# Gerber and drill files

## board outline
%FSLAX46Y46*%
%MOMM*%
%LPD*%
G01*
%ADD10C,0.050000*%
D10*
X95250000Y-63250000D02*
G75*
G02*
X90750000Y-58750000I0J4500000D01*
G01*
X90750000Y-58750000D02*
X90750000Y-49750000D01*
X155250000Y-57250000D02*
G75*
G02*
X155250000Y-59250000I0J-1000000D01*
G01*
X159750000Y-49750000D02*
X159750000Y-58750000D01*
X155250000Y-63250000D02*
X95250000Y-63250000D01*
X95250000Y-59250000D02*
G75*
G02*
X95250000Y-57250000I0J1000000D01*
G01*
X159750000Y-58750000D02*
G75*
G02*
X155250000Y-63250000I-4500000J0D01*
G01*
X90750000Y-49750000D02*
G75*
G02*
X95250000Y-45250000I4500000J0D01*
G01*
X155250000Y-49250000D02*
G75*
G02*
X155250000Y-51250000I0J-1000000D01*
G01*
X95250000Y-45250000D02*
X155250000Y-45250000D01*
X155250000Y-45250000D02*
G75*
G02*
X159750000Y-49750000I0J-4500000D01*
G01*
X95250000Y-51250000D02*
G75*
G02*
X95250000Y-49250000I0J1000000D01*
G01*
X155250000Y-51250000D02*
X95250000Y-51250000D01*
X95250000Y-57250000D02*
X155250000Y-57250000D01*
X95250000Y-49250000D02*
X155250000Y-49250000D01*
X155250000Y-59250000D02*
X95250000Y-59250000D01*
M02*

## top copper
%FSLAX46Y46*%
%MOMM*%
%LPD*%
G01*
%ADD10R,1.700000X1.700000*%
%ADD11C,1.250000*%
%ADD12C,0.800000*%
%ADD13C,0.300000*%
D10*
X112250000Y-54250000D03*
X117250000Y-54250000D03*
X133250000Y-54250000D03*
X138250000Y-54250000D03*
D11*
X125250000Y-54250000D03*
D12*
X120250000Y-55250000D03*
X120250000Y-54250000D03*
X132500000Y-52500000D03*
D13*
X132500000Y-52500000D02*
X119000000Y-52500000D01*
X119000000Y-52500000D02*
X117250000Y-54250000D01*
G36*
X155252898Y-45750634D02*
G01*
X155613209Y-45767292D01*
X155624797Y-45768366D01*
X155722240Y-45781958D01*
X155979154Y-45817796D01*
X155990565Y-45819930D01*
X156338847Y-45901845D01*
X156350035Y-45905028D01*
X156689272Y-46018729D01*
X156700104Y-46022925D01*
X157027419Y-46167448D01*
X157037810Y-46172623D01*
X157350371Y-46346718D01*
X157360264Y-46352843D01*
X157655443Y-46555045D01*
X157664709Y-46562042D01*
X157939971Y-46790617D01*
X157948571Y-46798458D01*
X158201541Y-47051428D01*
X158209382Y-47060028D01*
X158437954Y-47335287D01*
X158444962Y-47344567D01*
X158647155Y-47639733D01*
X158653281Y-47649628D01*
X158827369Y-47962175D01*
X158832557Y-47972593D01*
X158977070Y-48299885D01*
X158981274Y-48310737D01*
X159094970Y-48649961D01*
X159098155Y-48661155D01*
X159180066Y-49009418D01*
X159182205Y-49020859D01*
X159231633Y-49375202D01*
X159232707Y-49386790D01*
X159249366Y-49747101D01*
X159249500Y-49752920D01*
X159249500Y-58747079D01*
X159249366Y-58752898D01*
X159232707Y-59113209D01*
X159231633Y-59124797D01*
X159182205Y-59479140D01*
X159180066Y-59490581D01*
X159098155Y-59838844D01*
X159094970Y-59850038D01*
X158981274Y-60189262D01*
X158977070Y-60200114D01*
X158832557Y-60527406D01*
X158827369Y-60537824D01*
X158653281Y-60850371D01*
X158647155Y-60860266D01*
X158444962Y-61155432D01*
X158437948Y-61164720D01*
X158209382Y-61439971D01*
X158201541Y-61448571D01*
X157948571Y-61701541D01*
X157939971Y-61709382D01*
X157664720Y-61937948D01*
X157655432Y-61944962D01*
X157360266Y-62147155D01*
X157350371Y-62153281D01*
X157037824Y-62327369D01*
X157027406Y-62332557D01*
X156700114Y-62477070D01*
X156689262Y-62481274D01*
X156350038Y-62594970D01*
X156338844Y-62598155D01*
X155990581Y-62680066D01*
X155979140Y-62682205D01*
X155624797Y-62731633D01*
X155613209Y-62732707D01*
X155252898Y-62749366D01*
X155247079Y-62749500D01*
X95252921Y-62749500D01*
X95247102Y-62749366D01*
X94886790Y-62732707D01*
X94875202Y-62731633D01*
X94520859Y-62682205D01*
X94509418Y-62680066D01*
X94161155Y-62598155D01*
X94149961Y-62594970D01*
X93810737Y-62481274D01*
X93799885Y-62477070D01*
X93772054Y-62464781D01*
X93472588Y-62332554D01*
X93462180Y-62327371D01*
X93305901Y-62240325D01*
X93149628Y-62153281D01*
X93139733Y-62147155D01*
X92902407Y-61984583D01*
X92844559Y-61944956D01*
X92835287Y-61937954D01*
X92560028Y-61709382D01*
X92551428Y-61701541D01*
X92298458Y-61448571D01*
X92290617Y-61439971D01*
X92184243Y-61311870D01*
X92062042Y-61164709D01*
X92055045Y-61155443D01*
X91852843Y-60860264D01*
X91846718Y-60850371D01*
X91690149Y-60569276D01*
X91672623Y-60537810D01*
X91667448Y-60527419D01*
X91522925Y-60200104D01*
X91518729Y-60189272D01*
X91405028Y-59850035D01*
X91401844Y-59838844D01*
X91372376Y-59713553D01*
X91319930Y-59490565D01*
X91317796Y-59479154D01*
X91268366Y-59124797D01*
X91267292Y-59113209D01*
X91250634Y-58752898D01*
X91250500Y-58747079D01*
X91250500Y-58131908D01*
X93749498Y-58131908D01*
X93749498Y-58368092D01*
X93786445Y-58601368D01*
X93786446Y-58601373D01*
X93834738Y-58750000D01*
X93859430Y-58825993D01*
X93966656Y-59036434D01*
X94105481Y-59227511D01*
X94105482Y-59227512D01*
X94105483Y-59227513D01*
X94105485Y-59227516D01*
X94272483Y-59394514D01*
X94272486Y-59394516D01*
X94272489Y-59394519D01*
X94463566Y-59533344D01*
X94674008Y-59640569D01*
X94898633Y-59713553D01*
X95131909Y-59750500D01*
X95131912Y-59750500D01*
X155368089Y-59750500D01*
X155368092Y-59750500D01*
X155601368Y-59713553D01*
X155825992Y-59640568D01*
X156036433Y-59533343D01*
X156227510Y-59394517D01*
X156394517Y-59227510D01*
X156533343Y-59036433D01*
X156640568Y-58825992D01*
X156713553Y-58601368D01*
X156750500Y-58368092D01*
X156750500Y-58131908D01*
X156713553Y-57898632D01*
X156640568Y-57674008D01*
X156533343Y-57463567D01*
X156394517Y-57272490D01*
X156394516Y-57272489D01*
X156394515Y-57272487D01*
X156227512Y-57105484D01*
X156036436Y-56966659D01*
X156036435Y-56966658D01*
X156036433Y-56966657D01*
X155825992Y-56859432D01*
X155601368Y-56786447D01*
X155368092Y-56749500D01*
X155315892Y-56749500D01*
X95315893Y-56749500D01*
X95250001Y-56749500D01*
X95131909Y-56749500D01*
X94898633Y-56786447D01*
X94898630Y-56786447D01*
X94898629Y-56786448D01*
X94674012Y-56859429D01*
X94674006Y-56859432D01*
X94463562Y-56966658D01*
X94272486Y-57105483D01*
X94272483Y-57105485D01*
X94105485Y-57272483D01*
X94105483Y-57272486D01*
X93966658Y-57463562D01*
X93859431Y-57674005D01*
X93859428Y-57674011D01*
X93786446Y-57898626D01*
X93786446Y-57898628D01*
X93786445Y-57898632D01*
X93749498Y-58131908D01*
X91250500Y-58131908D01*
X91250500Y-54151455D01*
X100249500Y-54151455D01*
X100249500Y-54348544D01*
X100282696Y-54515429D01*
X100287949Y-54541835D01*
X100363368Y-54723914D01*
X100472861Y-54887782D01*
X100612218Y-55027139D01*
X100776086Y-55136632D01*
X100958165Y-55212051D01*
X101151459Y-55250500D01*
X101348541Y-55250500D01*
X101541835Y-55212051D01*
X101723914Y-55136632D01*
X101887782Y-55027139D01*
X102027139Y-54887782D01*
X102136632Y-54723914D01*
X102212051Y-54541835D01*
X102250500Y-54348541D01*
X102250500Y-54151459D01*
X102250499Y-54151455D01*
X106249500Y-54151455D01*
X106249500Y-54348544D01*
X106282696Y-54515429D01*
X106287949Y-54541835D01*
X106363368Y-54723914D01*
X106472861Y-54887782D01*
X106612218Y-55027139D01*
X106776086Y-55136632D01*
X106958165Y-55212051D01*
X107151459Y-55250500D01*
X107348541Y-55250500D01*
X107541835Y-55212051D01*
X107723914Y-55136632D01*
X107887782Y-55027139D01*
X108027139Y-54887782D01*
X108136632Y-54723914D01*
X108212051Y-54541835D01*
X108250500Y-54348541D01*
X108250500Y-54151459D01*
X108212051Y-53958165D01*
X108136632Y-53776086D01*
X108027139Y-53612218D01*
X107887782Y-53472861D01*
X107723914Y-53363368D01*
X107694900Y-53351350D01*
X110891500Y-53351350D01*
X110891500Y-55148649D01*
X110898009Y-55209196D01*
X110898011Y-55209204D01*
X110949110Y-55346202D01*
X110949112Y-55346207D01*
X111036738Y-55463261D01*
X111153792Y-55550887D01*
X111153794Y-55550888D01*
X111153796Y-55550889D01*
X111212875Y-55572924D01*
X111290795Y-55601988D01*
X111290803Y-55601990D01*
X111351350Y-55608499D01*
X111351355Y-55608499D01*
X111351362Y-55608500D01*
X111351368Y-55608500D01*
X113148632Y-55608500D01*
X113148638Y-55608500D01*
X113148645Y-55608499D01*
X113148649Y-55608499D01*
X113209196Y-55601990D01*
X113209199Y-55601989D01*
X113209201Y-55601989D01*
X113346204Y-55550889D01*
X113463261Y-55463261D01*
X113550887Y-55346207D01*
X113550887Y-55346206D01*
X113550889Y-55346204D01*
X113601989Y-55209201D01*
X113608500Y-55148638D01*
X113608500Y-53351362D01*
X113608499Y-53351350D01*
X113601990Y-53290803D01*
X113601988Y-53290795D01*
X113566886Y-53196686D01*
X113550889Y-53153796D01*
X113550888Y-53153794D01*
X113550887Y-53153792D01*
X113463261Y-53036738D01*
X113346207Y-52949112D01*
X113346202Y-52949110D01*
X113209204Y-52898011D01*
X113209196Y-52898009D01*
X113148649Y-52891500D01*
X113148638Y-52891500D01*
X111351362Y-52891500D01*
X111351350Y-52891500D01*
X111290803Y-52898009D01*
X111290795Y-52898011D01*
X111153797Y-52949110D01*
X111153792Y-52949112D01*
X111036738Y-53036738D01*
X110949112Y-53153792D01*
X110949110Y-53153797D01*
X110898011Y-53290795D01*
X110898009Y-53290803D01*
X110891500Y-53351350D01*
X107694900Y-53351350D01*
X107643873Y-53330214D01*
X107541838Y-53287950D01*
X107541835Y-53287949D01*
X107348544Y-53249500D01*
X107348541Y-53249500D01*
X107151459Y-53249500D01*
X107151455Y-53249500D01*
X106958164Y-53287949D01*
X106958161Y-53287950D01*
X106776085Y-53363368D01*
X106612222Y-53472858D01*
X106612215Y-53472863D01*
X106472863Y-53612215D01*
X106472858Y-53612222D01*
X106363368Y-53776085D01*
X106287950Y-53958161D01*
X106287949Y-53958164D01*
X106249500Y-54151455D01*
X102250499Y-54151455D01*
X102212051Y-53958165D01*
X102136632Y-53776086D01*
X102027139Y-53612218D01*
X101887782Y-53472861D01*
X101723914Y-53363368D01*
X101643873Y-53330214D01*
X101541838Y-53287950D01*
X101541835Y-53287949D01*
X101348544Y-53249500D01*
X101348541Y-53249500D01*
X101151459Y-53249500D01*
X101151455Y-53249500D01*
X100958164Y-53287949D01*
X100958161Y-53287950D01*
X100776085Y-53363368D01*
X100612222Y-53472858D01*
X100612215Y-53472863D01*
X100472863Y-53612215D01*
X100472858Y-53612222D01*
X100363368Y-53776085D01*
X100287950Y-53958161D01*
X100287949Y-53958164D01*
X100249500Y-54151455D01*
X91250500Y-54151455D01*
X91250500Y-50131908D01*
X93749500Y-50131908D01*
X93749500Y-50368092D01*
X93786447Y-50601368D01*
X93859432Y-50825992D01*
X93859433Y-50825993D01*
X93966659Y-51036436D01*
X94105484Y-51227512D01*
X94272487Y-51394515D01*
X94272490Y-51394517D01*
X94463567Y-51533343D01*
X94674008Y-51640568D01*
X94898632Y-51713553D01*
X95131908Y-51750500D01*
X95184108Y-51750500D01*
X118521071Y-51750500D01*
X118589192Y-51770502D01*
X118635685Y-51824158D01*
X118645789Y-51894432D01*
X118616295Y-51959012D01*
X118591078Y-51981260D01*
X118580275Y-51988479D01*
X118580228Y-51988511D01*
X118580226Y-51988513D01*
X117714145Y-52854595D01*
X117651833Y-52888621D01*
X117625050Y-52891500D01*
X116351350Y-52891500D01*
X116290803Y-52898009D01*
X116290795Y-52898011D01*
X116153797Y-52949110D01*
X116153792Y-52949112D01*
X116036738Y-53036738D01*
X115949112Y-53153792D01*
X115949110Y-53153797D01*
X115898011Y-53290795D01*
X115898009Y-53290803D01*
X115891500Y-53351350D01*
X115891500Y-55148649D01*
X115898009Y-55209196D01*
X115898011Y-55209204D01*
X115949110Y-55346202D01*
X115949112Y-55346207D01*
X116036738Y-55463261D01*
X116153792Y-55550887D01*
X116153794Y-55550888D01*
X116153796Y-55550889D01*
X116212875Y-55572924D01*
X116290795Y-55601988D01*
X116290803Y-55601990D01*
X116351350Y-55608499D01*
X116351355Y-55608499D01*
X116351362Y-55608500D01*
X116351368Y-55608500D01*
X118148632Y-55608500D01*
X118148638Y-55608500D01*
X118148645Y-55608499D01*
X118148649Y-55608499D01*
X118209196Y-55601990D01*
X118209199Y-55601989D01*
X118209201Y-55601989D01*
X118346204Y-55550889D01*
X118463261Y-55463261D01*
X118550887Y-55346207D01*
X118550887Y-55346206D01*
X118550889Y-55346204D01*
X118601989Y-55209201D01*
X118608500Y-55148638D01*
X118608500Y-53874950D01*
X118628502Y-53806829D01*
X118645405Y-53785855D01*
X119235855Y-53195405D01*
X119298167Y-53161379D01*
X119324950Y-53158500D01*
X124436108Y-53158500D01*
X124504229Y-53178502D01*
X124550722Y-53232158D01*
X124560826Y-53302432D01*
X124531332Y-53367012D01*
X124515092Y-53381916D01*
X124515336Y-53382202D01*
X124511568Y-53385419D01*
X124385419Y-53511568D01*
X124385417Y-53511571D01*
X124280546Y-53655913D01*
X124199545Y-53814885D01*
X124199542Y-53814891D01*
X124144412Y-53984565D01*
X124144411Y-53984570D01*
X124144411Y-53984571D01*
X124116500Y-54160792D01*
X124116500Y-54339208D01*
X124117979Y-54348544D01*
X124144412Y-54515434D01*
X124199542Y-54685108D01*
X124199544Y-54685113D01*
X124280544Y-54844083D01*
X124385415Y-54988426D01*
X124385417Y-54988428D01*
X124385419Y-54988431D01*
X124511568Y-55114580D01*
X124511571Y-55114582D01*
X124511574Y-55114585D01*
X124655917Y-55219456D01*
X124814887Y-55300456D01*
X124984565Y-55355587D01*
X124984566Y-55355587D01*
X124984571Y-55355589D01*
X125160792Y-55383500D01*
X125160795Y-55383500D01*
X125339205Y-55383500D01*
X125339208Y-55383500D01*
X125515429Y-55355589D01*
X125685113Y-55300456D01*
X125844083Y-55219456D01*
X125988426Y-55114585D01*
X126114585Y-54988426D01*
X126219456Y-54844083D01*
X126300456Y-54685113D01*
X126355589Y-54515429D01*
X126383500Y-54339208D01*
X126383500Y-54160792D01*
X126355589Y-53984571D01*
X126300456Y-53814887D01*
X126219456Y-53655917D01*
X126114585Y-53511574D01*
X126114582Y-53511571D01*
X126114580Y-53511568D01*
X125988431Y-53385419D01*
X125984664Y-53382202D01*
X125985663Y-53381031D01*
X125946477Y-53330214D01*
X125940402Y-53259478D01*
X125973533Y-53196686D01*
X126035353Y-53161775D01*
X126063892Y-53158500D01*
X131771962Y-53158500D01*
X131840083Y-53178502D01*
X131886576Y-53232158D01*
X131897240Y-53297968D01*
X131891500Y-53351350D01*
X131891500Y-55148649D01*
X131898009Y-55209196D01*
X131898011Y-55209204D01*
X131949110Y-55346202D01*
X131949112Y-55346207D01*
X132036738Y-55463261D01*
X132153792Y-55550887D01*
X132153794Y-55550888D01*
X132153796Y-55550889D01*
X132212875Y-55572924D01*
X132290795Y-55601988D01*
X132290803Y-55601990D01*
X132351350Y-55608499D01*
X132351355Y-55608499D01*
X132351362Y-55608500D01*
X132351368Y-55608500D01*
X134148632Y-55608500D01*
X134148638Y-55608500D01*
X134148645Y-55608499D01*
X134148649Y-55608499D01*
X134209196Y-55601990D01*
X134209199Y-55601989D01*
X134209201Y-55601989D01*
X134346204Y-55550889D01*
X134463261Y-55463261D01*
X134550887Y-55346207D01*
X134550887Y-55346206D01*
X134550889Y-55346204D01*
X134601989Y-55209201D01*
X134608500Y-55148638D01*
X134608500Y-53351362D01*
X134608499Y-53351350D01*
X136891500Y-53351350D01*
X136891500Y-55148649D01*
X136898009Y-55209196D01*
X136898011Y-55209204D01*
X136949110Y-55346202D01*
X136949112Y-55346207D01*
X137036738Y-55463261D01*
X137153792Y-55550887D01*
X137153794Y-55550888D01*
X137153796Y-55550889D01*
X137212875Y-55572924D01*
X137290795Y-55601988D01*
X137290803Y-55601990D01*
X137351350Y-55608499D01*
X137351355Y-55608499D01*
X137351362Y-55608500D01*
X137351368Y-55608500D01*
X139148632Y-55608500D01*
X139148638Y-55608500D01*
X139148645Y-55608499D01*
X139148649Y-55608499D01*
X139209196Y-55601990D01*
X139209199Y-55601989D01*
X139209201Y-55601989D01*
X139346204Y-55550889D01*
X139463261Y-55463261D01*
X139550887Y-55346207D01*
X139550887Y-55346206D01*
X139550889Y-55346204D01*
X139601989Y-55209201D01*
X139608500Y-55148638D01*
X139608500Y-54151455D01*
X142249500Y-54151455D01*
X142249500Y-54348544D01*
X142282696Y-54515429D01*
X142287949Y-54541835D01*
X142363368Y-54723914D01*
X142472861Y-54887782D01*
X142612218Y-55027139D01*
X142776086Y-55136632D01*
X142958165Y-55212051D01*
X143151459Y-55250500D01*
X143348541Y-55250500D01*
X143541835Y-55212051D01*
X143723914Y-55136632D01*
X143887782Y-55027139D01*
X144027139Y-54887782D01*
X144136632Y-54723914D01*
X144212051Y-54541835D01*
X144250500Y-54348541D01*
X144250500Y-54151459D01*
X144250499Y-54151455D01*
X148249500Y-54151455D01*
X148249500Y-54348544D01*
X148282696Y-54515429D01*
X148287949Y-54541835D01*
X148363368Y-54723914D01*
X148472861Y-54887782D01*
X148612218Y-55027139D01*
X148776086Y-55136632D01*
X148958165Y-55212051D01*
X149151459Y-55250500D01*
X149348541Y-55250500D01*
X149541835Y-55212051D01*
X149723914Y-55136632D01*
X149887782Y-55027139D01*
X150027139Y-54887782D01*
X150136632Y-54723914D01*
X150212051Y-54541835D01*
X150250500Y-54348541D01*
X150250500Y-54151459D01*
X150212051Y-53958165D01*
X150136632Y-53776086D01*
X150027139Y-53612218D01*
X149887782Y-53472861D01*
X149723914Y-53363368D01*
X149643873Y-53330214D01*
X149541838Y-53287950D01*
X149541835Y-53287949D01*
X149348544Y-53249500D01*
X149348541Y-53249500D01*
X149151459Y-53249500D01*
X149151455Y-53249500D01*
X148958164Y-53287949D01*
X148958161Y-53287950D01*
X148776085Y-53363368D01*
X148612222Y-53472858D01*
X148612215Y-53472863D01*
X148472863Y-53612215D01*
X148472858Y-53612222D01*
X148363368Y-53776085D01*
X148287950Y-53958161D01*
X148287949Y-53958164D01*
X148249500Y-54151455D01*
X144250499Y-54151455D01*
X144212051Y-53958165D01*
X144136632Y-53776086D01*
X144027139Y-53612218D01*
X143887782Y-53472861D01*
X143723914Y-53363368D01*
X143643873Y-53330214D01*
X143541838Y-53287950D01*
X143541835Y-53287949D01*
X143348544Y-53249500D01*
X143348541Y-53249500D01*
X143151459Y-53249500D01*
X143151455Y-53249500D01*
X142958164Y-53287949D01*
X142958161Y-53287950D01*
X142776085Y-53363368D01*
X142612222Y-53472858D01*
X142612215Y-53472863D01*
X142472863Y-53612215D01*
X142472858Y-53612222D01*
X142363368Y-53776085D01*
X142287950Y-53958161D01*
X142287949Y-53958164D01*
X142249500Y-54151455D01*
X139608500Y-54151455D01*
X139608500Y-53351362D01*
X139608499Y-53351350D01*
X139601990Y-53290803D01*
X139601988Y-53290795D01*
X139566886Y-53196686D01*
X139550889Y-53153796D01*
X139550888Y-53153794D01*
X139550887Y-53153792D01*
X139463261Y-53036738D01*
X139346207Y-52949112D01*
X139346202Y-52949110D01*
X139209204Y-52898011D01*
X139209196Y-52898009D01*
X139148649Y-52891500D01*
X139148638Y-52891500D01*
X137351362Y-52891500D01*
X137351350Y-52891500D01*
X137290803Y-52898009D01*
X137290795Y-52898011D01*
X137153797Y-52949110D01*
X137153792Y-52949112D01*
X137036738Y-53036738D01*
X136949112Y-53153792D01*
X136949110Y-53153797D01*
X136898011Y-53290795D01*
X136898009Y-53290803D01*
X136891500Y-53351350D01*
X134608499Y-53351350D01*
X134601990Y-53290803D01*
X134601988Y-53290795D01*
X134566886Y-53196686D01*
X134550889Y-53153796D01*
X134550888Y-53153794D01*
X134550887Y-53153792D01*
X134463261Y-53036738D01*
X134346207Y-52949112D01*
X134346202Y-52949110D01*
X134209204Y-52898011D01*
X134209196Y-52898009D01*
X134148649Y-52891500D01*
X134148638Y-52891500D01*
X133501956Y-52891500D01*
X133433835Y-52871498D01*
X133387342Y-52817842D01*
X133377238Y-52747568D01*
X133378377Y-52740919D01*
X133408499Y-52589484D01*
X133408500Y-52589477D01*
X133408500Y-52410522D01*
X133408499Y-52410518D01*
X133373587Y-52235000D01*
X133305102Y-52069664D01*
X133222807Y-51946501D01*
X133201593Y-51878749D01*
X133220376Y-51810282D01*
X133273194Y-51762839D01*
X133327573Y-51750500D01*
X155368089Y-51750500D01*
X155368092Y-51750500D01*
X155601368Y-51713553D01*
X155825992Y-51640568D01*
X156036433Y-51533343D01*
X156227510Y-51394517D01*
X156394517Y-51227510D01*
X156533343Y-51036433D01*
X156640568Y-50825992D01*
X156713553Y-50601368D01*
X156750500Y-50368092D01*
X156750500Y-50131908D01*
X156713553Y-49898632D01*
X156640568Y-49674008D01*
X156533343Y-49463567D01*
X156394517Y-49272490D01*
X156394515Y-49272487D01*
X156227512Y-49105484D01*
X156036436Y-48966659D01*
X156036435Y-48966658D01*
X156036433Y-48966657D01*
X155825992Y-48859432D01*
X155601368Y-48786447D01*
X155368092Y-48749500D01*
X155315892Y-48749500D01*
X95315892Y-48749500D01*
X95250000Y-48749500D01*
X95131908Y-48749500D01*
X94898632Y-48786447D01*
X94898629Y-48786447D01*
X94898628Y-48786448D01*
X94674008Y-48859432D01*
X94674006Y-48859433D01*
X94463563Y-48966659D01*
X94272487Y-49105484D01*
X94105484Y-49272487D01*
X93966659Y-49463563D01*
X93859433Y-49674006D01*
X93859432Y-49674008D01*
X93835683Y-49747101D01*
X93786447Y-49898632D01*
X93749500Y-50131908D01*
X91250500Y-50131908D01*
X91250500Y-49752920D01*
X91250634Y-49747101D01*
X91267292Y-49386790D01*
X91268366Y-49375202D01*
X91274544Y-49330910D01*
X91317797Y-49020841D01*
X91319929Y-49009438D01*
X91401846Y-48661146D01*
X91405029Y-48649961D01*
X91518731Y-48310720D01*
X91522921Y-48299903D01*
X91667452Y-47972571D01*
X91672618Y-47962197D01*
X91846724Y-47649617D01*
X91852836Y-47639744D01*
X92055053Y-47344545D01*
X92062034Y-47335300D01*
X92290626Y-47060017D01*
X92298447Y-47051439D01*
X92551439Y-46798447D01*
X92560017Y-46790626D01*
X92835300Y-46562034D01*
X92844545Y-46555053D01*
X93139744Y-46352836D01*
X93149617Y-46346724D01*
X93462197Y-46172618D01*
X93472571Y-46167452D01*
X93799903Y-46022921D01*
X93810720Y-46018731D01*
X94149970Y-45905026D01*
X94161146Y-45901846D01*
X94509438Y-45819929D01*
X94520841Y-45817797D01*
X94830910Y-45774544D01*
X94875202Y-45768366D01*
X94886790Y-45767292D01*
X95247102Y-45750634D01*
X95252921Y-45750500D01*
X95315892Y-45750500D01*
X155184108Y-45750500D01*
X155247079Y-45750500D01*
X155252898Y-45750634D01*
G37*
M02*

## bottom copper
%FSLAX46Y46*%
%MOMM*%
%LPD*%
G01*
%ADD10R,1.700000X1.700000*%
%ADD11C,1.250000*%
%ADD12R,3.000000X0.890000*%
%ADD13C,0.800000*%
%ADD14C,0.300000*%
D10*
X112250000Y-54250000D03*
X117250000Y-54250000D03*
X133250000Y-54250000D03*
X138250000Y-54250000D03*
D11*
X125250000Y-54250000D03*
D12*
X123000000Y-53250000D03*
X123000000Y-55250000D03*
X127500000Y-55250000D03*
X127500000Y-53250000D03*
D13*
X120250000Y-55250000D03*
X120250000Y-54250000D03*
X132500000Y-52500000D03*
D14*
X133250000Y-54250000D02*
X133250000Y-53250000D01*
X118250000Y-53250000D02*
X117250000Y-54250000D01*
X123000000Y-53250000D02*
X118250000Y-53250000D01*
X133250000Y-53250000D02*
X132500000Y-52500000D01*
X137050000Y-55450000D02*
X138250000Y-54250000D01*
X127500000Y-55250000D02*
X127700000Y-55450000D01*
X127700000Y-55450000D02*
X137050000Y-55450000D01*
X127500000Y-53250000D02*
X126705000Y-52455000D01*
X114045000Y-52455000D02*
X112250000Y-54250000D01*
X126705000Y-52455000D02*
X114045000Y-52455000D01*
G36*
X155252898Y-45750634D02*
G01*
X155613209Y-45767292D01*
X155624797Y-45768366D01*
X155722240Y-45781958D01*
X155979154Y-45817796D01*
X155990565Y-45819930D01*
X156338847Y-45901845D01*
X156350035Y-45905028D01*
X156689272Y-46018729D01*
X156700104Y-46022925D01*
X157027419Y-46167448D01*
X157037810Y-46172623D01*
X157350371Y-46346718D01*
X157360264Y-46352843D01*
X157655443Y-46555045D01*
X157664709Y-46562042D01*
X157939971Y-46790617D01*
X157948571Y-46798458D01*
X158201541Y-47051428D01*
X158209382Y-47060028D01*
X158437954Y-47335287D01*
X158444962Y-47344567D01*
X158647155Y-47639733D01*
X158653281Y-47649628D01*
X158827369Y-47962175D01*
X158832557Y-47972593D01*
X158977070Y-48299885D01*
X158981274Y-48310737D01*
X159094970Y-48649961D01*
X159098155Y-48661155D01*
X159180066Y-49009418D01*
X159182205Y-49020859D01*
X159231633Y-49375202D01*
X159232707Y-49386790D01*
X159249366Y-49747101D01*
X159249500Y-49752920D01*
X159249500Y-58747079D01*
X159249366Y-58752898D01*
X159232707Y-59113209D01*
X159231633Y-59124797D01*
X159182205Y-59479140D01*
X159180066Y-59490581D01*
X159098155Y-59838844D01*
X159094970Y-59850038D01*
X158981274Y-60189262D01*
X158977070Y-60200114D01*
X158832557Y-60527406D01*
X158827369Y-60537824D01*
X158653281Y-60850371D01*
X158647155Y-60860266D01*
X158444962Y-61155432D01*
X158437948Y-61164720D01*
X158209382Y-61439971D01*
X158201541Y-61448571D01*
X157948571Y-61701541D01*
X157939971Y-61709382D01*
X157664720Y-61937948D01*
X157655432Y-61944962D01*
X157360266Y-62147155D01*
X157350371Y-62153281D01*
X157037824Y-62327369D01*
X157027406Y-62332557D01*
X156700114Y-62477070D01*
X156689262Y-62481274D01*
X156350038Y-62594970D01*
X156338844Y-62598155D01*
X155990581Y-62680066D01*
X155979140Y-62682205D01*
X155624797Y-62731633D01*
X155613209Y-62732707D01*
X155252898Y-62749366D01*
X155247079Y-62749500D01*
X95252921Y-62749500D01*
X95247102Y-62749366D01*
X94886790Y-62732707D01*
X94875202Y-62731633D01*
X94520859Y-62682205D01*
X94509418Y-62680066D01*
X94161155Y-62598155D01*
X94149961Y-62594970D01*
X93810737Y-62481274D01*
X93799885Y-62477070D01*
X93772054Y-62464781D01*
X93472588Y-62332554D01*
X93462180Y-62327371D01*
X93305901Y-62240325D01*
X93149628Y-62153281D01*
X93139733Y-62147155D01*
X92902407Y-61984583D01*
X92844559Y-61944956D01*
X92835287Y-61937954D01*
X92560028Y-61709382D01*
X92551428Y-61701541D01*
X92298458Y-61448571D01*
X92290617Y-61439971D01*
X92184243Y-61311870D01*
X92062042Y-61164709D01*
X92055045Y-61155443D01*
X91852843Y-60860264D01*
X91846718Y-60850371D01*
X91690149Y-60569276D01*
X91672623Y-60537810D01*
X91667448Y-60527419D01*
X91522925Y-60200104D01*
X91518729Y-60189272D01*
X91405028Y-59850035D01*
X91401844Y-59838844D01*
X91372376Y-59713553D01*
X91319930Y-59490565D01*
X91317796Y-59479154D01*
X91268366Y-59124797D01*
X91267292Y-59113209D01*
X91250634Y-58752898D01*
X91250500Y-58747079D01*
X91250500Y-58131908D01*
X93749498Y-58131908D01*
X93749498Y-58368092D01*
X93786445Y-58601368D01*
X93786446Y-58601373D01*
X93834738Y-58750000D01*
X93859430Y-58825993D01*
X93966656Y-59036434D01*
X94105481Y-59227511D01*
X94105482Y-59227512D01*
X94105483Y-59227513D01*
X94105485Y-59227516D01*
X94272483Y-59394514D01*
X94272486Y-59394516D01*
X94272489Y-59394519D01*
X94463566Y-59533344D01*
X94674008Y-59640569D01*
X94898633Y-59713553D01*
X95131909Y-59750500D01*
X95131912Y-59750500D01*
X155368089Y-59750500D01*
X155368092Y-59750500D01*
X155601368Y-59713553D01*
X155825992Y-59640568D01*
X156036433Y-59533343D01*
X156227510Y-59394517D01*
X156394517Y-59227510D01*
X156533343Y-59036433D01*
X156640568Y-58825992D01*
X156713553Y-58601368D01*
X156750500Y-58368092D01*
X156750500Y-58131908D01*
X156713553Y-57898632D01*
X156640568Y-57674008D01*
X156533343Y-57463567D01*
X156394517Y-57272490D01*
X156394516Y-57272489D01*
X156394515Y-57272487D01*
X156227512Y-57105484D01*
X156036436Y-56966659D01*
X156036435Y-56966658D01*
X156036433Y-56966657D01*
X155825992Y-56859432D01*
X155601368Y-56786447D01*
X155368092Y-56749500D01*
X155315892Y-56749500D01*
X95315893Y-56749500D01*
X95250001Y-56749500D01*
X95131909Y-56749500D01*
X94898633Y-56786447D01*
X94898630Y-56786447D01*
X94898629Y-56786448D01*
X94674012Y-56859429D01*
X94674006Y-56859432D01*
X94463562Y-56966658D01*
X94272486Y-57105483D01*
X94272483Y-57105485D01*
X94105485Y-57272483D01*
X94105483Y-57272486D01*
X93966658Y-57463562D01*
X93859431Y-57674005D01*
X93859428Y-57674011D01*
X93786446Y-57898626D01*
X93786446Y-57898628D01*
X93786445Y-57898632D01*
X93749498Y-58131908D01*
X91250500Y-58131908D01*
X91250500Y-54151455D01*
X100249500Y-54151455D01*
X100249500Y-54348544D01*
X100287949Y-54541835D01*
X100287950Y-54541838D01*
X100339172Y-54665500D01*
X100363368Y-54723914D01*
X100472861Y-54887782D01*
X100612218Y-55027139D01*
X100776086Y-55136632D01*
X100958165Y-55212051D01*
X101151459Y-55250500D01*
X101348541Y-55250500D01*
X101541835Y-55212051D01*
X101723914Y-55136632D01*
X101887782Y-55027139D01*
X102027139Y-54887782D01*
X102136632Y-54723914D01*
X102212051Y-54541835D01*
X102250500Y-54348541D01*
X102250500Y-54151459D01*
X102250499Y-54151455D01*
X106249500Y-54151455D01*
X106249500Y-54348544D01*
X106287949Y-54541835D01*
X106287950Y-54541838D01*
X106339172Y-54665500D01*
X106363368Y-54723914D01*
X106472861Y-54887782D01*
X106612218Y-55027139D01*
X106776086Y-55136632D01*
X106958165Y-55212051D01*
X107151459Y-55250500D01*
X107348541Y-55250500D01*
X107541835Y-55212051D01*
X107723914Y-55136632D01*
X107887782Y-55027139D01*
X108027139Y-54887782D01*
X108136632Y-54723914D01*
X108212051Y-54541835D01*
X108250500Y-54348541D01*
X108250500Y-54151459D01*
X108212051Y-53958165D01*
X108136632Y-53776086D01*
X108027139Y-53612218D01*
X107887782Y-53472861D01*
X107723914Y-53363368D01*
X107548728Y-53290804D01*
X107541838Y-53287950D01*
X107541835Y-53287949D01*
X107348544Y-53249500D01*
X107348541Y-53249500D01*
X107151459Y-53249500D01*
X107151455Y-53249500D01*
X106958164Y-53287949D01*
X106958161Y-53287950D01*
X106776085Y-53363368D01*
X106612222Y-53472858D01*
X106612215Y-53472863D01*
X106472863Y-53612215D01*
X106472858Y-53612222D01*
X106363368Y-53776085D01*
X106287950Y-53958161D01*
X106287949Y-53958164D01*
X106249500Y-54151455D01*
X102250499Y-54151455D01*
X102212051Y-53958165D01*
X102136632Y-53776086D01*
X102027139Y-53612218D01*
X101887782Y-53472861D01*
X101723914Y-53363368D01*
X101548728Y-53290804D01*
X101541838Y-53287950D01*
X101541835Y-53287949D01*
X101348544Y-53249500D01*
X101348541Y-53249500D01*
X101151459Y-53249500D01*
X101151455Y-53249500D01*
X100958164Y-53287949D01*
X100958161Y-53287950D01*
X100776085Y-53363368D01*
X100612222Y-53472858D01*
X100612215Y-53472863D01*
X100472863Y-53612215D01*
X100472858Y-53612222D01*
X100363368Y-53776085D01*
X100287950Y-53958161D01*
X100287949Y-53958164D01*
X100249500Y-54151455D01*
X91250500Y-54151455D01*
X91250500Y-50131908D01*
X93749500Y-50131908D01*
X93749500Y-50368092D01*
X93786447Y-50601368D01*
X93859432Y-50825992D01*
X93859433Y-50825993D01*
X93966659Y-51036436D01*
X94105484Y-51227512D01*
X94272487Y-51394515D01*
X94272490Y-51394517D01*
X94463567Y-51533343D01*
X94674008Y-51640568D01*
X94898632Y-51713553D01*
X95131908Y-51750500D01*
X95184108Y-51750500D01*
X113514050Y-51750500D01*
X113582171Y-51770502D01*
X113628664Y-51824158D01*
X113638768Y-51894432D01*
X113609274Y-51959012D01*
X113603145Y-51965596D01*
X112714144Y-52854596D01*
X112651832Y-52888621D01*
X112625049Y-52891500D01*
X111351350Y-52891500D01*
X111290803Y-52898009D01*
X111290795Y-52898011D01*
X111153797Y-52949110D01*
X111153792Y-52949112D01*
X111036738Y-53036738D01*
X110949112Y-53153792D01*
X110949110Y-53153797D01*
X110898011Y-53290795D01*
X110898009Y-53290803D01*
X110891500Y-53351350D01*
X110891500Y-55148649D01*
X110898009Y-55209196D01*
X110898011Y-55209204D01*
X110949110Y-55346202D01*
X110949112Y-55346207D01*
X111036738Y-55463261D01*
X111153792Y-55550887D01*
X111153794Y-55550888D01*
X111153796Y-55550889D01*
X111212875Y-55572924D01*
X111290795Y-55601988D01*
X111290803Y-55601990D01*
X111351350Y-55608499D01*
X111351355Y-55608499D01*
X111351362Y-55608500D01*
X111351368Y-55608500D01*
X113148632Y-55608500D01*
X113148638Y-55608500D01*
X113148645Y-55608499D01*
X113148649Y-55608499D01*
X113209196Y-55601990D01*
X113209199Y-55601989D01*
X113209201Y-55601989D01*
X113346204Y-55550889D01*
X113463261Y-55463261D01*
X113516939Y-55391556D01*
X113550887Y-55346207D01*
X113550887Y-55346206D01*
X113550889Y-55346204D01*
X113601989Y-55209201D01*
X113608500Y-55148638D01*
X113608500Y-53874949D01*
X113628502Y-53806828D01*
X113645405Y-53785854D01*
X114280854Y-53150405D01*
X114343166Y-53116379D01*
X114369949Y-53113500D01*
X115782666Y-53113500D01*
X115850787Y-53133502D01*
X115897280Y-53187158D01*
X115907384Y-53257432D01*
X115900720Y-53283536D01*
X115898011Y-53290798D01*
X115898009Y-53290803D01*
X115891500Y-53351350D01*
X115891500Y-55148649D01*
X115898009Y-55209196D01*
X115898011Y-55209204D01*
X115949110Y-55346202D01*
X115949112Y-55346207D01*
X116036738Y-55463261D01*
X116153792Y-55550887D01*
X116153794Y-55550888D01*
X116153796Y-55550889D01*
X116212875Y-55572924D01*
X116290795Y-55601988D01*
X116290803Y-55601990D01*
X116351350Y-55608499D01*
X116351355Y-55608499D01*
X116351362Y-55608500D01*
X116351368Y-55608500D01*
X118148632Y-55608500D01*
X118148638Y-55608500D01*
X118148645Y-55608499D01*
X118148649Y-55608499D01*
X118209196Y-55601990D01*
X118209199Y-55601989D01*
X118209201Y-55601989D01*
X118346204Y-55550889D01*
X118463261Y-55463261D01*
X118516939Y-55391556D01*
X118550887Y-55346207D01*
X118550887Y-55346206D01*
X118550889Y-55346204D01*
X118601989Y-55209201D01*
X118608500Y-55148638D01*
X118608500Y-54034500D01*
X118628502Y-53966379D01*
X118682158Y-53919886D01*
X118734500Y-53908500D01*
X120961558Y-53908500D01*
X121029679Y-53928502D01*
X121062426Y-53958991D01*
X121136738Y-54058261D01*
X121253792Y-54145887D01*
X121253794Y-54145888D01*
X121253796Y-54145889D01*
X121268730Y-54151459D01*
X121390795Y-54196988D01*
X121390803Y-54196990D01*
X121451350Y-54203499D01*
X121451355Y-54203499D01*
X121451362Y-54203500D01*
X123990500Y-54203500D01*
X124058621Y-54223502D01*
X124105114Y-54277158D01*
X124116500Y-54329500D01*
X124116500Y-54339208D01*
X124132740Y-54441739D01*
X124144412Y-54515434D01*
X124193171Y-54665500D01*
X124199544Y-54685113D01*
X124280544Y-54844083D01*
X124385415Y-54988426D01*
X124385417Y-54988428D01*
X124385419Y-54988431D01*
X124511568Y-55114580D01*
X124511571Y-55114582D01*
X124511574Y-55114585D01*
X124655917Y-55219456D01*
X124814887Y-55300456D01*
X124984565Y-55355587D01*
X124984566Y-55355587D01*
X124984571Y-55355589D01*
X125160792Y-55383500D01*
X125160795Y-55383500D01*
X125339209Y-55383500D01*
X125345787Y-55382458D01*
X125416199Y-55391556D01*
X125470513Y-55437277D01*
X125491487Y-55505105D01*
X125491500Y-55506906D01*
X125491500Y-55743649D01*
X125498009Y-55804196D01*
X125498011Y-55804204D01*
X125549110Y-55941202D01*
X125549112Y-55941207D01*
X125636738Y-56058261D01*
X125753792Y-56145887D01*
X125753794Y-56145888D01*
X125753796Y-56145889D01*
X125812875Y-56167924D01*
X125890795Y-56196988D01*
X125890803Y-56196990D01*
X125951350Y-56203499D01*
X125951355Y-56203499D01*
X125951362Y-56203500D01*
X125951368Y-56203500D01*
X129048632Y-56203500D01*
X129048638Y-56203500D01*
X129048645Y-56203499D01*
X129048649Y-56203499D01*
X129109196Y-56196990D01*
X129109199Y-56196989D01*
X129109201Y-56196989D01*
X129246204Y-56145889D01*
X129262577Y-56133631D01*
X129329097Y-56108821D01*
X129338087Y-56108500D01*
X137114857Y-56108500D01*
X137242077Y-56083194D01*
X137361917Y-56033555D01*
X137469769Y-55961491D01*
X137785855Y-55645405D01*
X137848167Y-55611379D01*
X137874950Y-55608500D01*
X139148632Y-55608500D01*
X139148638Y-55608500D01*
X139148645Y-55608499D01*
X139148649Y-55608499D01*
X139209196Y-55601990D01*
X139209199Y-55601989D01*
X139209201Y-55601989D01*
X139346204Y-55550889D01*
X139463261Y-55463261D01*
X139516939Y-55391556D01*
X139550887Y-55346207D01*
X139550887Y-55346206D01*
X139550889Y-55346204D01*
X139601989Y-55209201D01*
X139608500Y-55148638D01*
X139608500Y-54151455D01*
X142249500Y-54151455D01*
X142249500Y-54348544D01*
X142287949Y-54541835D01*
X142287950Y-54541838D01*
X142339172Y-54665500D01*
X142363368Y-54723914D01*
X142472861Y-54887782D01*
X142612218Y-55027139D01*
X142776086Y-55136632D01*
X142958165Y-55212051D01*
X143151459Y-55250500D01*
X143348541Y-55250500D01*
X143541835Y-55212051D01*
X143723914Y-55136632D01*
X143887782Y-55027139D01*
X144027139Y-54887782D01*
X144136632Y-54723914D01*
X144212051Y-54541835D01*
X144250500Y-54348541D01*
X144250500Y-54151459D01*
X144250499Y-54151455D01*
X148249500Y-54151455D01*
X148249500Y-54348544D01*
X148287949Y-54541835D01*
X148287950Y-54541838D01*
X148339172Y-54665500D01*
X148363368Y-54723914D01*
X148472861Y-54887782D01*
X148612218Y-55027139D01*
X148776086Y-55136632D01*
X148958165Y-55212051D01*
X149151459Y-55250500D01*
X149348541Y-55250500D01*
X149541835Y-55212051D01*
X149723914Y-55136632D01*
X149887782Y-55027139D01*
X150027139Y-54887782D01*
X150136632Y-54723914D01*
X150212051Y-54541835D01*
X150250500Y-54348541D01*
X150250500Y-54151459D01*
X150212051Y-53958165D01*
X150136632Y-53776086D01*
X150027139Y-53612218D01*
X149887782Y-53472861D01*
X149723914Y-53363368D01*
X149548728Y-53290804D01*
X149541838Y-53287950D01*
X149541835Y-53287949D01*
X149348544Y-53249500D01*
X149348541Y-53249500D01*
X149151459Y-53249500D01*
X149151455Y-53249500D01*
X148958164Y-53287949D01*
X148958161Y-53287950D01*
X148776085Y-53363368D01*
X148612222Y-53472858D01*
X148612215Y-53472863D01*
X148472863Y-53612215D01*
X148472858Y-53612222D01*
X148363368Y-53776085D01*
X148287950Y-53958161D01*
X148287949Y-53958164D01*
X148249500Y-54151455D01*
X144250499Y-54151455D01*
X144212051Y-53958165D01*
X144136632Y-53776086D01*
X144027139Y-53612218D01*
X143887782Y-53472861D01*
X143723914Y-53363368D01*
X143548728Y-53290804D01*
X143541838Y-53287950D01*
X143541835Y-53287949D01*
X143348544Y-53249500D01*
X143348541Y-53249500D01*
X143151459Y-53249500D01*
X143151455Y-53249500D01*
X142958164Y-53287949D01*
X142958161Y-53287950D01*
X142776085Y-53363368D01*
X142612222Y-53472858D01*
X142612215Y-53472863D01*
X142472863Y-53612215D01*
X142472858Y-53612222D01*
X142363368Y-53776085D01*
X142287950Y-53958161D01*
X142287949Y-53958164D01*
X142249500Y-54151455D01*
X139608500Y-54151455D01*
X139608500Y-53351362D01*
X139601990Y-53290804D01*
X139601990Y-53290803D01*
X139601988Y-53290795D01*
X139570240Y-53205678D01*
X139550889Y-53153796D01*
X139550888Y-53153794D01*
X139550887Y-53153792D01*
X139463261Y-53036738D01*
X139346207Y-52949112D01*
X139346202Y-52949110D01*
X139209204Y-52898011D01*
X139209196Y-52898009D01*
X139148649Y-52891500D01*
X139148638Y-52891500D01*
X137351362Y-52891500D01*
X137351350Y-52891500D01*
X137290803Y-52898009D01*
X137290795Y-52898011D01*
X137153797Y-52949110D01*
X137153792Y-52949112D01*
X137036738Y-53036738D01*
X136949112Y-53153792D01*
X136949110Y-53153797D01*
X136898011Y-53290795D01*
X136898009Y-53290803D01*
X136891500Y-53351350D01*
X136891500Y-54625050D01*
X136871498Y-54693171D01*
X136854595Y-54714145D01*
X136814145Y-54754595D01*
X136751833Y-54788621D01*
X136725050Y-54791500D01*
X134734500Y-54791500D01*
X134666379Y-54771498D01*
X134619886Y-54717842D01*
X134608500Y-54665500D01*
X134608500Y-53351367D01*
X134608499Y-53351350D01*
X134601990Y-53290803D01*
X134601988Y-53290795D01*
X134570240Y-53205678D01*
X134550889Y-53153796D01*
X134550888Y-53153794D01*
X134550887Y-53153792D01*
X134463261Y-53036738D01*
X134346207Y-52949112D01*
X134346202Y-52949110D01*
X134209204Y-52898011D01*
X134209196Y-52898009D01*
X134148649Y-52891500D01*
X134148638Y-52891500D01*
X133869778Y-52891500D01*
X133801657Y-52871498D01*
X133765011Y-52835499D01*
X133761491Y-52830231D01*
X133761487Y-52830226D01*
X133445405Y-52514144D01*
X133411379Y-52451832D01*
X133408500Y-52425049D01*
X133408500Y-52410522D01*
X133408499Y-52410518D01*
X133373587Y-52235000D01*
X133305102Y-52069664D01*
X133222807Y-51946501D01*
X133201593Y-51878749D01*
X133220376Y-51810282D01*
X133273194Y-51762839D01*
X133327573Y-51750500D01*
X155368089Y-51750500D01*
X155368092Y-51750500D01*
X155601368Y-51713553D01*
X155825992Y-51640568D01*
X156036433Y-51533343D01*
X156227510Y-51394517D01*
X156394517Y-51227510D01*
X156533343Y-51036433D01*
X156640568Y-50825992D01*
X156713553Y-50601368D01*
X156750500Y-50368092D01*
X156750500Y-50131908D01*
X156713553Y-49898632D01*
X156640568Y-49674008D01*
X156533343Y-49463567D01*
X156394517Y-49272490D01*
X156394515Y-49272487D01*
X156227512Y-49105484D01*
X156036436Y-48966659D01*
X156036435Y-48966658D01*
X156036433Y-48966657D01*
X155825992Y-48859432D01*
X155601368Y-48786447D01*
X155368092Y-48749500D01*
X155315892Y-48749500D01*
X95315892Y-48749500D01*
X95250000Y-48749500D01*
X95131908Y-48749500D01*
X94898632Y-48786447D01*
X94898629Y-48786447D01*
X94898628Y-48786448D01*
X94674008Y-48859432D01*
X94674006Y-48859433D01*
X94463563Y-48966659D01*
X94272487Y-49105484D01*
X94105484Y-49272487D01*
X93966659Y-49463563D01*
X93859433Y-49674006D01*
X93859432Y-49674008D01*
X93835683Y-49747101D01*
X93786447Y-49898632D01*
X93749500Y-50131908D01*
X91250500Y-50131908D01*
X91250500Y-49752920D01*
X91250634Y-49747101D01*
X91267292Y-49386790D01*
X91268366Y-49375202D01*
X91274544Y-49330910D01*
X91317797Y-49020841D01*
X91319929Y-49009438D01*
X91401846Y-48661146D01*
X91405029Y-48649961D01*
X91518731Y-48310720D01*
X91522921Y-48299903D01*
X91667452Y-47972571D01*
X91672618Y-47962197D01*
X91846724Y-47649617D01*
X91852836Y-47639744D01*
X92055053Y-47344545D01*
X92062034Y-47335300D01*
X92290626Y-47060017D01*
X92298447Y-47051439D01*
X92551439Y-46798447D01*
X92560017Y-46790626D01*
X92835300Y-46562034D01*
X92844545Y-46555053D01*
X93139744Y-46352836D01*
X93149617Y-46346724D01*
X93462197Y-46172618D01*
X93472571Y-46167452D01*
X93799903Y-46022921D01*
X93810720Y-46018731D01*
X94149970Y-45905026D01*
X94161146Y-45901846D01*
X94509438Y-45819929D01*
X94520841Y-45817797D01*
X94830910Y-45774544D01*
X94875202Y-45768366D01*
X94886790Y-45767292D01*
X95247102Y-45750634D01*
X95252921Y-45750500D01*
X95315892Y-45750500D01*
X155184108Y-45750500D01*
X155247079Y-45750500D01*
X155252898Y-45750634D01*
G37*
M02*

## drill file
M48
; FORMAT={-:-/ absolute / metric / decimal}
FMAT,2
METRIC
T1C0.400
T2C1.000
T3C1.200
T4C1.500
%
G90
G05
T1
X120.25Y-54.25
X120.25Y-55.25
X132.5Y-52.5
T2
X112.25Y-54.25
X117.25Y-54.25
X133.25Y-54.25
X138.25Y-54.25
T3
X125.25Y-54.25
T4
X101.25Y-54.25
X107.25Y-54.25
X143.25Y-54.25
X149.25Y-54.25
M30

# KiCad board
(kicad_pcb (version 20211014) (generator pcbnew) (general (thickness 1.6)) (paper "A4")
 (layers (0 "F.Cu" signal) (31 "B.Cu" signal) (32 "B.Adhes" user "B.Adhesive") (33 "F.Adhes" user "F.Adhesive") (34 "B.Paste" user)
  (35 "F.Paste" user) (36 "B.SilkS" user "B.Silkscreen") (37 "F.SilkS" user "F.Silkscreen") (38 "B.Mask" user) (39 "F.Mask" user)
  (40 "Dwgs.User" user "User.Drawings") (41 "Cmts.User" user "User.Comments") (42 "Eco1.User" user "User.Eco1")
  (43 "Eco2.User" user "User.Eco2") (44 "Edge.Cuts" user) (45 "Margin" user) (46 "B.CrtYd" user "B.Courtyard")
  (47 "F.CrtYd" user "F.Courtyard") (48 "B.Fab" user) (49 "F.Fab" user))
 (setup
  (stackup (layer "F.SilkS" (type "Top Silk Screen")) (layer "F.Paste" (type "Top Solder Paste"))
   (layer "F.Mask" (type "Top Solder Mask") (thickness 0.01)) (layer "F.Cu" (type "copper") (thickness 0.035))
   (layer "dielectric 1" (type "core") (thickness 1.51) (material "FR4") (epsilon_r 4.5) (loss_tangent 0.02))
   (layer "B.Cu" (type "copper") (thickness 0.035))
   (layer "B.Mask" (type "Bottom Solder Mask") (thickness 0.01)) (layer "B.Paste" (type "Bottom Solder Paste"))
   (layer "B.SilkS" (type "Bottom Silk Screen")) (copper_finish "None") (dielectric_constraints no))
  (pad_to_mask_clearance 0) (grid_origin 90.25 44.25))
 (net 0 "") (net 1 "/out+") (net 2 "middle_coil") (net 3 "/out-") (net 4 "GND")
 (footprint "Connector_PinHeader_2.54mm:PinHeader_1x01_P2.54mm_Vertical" (layer "F.Cu") (at 112.25 54.25 -90)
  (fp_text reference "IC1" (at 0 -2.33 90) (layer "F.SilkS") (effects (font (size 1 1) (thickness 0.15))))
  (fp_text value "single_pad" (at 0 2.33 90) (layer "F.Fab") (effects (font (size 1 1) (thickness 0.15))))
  (pad "1" thru_hole rect (at 0 0 270) (size 1.7 1.7) (drill 1) (layers *.Cu *.Mask) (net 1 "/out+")))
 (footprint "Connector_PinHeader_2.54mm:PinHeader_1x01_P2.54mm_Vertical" (layer "F.Cu") (at 117.25 54.25 -90)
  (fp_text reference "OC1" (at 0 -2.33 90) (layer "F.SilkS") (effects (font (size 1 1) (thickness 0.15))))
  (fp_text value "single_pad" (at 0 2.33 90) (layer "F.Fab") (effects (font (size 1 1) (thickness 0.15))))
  (pad "1" thru_hole rect (at 0 0 270) (size 1.7 1.7) (drill 1) (layers *.Cu *.Mask) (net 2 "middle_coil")))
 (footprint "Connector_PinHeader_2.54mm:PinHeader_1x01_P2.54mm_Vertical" (layer "F.Cu") (at 133.25 54.25 90)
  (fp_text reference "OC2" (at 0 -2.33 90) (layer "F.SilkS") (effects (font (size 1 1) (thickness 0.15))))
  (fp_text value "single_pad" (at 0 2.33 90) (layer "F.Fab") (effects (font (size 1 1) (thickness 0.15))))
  (pad "1" thru_hole rect (at 0 0 90) (size 1.7 1.7) (drill 1) (layers *.Cu *.Mask) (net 2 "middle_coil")))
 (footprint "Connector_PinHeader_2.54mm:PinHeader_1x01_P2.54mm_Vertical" (layer "F.Cu") (at 138.25 54.25 90)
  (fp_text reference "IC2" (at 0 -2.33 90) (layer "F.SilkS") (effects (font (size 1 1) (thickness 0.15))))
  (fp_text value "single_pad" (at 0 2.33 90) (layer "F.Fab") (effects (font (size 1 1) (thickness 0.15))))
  (pad "1" thru_hole rect (at 0 0 90) (size 1.7 1.7) (drill 1) (layers *.Cu *.Mask) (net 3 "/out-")))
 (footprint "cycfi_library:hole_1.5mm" (layer "F.Cu") (at 107.25 54.25)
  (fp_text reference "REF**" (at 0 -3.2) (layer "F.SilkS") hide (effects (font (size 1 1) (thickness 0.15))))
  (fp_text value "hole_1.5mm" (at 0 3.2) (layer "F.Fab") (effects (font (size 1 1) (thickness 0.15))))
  (pad "" np_thru_hole circle locked (at 0 0) (size 1.5 1.5) (drill 1.5) (layers *.Cu *.Mask)))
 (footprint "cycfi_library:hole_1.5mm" (layer "F.Cu") (at 143.25 54.25)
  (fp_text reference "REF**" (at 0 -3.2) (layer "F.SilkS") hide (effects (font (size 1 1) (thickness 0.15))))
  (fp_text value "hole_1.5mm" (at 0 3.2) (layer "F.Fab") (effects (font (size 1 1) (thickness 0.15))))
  (pad "" np_thru_hole circle locked (at 0 0) (size 1.5 1.5) (drill 1.5) (layers *.Cu *.Mask)))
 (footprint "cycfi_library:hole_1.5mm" (layer "F.Cu") (at 149.25 54.25)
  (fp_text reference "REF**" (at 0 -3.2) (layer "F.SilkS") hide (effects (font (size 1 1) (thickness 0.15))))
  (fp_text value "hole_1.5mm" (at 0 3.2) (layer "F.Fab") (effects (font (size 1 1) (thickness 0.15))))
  (pad "" np_thru_hole circle locked (at 0 0) (size 1.5 1.5) (drill 1.5) (layers *.Cu *.Mask)))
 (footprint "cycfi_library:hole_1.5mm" (layer "F.Cu") (at 101.25 54.25)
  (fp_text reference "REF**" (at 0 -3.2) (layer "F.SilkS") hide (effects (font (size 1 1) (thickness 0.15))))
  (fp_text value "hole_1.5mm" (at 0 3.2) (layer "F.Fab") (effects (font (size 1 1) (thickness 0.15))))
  (pad "" np_thru_hole circle locked (at 0 0) (size 1.5 1.5) (drill 1.5) (layers *.Cu *.Mask)))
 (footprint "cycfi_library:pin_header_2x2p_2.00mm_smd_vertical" (layer "B.Cu") (at 125.25 54.25 180)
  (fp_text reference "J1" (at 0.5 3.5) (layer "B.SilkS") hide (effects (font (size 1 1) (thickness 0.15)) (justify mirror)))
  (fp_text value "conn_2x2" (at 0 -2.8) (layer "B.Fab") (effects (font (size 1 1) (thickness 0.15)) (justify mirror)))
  (pad "" np_thru_hole circle (at 0 0 180) (size 1.25 1.25) (drill 1.2) (layers F&B.Cu *.Mask))
  (pad "1" smd rect (at 2.25 1 180) (size 3 0.89) (layers "B.Cu" "B.Paste" "B.Mask") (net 2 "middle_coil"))
  (pad "2" smd rect (at 2.25 -1 180) (size 3 0.89) (layers "B.Cu" "B.Paste" "B.Mask") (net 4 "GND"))
  (pad "3" smd rect (at -2.25 -1 180) (size 3 0.89) (layers "B.Cu" "B.Paste" "B.Mask") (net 3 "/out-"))
  (pad "4" smd rect (at -2.25 1 180) (size 3 0.89) (layers "B.Cu" "B.Paste" "B.Mask") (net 1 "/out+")))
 (gr_arc (start 95.25 63.25) (mid 92.068019 61.931981) (end 90.75 58.75) (layer "Edge.Cuts") (width 0.05))
 (gr_line (start 90.75 58.75) (end 90.75 49.75) (layer "Edge.Cuts") (width 0.05))
 (gr_arc (start 155.25 57.25) (mid 156.25 58.25) (end 155.25 59.25) (layer "Edge.Cuts") (width 0.05))
 (gr_line (start 159.75 49.75) (end 159.75 58.75) (layer "Edge.Cuts") (width 0.05))
 (gr_line (start 155.25 63.25) (end 95.25 63.25) (layer "Edge.Cuts") (width 0.05))
 (gr_arc (start 95.25 59.25) (mid 94.249998 58.25) (end 95.25 57.25) (layer "Edge.Cuts") (width 0.05))
 (gr_arc (start 159.75 58.75) (mid 158.431981 61.931981) (end 155.25 63.25) (layer "Edge.Cuts") (width 0.05))
 (gr_arc (start 90.75 49.75) (mid 92.068019 46.568019) (end 95.25 45.25) (layer "Edge.Cuts") (width 0.05))
 (gr_arc (start 155.25 49.25) (mid 156.25 50.25) (end 155.25 51.25) (layer "Edge.Cuts") (width 0.05))
 (gr_line (start 95.25 45.25) (end 155.25 45.25) (layer "Edge.Cuts") (width 0.05))
 (gr_arc (start 155.25 45.25) (mid 158.431981 46.568019) (end 159.75 49.75) (layer "Edge.Cuts") (width 0.05))
 (gr_arc (start 95.25 51.25) (mid 94.25 50.25) (end 95.25 49.25) (layer "Edge.Cuts") (width 0.05))
 (gr_line (start 155.25 51.25) (end 95.25 51.25) (layer "Edge.Cuts") (width 0.05))
 (gr_line (start 95.25 57.25) (end 155.25 57.25) (layer "Edge.Cuts") (width 0.05))
 (gr_line (start 95.25 49.25) (end 155.25 49.25) (layer "Edge.Cuts") (width 0.05))
 (gr_line (start 155.25 59.25) (end 95.25 59.25) (layer "Edge.Cuts") (width 0.05))
 (via (at 120.25 55.25) (size 0.8) (drill 0.4) (layers "F.Cu" "B.Cu") (free) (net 4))
 (via (at 120.25 54.25) (size 0.8) (drill 0.4) (layers "F.Cu" "B.Cu") (free) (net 4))
 (segment (start 132.5 52.5) (end 119 52.5) (width 0.3) (layer "F.Cu") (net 2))
 (segment (start 119 52.5) (end 117.25 54.25) (width 0.3) (layer "F.Cu") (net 2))
 (via (at 132.5 52.5) (size 0.8) (drill 0.4) (layers "F.Cu" "B.Cu") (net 2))
 (segment (start 133.25 54.25) (end 133.25 53.25) (width 0.3) (layer "B.Cu") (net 2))
 (segment (start 118.25 53.25) (end 117.25 54.25) (width 0.3) (layer "B.Cu") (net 2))
 (segment (start 123 53.25) (end 118.25 53.25) (width 0.3) (layer "B.Cu") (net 2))
 (segment (start 133.25 53.25) (end 132.5 52.5) (width 0.3) (layer "B.Cu") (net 2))
 (segment (start 137.05 55.45) (end 138.25 54.25) (width 0.3) (layer "B.Cu") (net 3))
 (segment (start 127.5 55.25) (end 127.7 55.45) (width 0.3) (layer "B.Cu") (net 3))
 (segment (start 127.7 55.45) (end 137.05 55.45) (width 0.3) (layer "B.Cu") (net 3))
 (segment (start 127.5 53.25) (end 126.705 52.455) (width 0.3) (layer "B.Cu") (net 1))
 (segment (start 114.045 52.455) (end 112.25 54.25) (width 0.3) (layer "B.Cu") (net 1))
 (segment (start 126.705 52.455) (end 114.045 52.455) (width 0.3) (layer "B.Cu") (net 1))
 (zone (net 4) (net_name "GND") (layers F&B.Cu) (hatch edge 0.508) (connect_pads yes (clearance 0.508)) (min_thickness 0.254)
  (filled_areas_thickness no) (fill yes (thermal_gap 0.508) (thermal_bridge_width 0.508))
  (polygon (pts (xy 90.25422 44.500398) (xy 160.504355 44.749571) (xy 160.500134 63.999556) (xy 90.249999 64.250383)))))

